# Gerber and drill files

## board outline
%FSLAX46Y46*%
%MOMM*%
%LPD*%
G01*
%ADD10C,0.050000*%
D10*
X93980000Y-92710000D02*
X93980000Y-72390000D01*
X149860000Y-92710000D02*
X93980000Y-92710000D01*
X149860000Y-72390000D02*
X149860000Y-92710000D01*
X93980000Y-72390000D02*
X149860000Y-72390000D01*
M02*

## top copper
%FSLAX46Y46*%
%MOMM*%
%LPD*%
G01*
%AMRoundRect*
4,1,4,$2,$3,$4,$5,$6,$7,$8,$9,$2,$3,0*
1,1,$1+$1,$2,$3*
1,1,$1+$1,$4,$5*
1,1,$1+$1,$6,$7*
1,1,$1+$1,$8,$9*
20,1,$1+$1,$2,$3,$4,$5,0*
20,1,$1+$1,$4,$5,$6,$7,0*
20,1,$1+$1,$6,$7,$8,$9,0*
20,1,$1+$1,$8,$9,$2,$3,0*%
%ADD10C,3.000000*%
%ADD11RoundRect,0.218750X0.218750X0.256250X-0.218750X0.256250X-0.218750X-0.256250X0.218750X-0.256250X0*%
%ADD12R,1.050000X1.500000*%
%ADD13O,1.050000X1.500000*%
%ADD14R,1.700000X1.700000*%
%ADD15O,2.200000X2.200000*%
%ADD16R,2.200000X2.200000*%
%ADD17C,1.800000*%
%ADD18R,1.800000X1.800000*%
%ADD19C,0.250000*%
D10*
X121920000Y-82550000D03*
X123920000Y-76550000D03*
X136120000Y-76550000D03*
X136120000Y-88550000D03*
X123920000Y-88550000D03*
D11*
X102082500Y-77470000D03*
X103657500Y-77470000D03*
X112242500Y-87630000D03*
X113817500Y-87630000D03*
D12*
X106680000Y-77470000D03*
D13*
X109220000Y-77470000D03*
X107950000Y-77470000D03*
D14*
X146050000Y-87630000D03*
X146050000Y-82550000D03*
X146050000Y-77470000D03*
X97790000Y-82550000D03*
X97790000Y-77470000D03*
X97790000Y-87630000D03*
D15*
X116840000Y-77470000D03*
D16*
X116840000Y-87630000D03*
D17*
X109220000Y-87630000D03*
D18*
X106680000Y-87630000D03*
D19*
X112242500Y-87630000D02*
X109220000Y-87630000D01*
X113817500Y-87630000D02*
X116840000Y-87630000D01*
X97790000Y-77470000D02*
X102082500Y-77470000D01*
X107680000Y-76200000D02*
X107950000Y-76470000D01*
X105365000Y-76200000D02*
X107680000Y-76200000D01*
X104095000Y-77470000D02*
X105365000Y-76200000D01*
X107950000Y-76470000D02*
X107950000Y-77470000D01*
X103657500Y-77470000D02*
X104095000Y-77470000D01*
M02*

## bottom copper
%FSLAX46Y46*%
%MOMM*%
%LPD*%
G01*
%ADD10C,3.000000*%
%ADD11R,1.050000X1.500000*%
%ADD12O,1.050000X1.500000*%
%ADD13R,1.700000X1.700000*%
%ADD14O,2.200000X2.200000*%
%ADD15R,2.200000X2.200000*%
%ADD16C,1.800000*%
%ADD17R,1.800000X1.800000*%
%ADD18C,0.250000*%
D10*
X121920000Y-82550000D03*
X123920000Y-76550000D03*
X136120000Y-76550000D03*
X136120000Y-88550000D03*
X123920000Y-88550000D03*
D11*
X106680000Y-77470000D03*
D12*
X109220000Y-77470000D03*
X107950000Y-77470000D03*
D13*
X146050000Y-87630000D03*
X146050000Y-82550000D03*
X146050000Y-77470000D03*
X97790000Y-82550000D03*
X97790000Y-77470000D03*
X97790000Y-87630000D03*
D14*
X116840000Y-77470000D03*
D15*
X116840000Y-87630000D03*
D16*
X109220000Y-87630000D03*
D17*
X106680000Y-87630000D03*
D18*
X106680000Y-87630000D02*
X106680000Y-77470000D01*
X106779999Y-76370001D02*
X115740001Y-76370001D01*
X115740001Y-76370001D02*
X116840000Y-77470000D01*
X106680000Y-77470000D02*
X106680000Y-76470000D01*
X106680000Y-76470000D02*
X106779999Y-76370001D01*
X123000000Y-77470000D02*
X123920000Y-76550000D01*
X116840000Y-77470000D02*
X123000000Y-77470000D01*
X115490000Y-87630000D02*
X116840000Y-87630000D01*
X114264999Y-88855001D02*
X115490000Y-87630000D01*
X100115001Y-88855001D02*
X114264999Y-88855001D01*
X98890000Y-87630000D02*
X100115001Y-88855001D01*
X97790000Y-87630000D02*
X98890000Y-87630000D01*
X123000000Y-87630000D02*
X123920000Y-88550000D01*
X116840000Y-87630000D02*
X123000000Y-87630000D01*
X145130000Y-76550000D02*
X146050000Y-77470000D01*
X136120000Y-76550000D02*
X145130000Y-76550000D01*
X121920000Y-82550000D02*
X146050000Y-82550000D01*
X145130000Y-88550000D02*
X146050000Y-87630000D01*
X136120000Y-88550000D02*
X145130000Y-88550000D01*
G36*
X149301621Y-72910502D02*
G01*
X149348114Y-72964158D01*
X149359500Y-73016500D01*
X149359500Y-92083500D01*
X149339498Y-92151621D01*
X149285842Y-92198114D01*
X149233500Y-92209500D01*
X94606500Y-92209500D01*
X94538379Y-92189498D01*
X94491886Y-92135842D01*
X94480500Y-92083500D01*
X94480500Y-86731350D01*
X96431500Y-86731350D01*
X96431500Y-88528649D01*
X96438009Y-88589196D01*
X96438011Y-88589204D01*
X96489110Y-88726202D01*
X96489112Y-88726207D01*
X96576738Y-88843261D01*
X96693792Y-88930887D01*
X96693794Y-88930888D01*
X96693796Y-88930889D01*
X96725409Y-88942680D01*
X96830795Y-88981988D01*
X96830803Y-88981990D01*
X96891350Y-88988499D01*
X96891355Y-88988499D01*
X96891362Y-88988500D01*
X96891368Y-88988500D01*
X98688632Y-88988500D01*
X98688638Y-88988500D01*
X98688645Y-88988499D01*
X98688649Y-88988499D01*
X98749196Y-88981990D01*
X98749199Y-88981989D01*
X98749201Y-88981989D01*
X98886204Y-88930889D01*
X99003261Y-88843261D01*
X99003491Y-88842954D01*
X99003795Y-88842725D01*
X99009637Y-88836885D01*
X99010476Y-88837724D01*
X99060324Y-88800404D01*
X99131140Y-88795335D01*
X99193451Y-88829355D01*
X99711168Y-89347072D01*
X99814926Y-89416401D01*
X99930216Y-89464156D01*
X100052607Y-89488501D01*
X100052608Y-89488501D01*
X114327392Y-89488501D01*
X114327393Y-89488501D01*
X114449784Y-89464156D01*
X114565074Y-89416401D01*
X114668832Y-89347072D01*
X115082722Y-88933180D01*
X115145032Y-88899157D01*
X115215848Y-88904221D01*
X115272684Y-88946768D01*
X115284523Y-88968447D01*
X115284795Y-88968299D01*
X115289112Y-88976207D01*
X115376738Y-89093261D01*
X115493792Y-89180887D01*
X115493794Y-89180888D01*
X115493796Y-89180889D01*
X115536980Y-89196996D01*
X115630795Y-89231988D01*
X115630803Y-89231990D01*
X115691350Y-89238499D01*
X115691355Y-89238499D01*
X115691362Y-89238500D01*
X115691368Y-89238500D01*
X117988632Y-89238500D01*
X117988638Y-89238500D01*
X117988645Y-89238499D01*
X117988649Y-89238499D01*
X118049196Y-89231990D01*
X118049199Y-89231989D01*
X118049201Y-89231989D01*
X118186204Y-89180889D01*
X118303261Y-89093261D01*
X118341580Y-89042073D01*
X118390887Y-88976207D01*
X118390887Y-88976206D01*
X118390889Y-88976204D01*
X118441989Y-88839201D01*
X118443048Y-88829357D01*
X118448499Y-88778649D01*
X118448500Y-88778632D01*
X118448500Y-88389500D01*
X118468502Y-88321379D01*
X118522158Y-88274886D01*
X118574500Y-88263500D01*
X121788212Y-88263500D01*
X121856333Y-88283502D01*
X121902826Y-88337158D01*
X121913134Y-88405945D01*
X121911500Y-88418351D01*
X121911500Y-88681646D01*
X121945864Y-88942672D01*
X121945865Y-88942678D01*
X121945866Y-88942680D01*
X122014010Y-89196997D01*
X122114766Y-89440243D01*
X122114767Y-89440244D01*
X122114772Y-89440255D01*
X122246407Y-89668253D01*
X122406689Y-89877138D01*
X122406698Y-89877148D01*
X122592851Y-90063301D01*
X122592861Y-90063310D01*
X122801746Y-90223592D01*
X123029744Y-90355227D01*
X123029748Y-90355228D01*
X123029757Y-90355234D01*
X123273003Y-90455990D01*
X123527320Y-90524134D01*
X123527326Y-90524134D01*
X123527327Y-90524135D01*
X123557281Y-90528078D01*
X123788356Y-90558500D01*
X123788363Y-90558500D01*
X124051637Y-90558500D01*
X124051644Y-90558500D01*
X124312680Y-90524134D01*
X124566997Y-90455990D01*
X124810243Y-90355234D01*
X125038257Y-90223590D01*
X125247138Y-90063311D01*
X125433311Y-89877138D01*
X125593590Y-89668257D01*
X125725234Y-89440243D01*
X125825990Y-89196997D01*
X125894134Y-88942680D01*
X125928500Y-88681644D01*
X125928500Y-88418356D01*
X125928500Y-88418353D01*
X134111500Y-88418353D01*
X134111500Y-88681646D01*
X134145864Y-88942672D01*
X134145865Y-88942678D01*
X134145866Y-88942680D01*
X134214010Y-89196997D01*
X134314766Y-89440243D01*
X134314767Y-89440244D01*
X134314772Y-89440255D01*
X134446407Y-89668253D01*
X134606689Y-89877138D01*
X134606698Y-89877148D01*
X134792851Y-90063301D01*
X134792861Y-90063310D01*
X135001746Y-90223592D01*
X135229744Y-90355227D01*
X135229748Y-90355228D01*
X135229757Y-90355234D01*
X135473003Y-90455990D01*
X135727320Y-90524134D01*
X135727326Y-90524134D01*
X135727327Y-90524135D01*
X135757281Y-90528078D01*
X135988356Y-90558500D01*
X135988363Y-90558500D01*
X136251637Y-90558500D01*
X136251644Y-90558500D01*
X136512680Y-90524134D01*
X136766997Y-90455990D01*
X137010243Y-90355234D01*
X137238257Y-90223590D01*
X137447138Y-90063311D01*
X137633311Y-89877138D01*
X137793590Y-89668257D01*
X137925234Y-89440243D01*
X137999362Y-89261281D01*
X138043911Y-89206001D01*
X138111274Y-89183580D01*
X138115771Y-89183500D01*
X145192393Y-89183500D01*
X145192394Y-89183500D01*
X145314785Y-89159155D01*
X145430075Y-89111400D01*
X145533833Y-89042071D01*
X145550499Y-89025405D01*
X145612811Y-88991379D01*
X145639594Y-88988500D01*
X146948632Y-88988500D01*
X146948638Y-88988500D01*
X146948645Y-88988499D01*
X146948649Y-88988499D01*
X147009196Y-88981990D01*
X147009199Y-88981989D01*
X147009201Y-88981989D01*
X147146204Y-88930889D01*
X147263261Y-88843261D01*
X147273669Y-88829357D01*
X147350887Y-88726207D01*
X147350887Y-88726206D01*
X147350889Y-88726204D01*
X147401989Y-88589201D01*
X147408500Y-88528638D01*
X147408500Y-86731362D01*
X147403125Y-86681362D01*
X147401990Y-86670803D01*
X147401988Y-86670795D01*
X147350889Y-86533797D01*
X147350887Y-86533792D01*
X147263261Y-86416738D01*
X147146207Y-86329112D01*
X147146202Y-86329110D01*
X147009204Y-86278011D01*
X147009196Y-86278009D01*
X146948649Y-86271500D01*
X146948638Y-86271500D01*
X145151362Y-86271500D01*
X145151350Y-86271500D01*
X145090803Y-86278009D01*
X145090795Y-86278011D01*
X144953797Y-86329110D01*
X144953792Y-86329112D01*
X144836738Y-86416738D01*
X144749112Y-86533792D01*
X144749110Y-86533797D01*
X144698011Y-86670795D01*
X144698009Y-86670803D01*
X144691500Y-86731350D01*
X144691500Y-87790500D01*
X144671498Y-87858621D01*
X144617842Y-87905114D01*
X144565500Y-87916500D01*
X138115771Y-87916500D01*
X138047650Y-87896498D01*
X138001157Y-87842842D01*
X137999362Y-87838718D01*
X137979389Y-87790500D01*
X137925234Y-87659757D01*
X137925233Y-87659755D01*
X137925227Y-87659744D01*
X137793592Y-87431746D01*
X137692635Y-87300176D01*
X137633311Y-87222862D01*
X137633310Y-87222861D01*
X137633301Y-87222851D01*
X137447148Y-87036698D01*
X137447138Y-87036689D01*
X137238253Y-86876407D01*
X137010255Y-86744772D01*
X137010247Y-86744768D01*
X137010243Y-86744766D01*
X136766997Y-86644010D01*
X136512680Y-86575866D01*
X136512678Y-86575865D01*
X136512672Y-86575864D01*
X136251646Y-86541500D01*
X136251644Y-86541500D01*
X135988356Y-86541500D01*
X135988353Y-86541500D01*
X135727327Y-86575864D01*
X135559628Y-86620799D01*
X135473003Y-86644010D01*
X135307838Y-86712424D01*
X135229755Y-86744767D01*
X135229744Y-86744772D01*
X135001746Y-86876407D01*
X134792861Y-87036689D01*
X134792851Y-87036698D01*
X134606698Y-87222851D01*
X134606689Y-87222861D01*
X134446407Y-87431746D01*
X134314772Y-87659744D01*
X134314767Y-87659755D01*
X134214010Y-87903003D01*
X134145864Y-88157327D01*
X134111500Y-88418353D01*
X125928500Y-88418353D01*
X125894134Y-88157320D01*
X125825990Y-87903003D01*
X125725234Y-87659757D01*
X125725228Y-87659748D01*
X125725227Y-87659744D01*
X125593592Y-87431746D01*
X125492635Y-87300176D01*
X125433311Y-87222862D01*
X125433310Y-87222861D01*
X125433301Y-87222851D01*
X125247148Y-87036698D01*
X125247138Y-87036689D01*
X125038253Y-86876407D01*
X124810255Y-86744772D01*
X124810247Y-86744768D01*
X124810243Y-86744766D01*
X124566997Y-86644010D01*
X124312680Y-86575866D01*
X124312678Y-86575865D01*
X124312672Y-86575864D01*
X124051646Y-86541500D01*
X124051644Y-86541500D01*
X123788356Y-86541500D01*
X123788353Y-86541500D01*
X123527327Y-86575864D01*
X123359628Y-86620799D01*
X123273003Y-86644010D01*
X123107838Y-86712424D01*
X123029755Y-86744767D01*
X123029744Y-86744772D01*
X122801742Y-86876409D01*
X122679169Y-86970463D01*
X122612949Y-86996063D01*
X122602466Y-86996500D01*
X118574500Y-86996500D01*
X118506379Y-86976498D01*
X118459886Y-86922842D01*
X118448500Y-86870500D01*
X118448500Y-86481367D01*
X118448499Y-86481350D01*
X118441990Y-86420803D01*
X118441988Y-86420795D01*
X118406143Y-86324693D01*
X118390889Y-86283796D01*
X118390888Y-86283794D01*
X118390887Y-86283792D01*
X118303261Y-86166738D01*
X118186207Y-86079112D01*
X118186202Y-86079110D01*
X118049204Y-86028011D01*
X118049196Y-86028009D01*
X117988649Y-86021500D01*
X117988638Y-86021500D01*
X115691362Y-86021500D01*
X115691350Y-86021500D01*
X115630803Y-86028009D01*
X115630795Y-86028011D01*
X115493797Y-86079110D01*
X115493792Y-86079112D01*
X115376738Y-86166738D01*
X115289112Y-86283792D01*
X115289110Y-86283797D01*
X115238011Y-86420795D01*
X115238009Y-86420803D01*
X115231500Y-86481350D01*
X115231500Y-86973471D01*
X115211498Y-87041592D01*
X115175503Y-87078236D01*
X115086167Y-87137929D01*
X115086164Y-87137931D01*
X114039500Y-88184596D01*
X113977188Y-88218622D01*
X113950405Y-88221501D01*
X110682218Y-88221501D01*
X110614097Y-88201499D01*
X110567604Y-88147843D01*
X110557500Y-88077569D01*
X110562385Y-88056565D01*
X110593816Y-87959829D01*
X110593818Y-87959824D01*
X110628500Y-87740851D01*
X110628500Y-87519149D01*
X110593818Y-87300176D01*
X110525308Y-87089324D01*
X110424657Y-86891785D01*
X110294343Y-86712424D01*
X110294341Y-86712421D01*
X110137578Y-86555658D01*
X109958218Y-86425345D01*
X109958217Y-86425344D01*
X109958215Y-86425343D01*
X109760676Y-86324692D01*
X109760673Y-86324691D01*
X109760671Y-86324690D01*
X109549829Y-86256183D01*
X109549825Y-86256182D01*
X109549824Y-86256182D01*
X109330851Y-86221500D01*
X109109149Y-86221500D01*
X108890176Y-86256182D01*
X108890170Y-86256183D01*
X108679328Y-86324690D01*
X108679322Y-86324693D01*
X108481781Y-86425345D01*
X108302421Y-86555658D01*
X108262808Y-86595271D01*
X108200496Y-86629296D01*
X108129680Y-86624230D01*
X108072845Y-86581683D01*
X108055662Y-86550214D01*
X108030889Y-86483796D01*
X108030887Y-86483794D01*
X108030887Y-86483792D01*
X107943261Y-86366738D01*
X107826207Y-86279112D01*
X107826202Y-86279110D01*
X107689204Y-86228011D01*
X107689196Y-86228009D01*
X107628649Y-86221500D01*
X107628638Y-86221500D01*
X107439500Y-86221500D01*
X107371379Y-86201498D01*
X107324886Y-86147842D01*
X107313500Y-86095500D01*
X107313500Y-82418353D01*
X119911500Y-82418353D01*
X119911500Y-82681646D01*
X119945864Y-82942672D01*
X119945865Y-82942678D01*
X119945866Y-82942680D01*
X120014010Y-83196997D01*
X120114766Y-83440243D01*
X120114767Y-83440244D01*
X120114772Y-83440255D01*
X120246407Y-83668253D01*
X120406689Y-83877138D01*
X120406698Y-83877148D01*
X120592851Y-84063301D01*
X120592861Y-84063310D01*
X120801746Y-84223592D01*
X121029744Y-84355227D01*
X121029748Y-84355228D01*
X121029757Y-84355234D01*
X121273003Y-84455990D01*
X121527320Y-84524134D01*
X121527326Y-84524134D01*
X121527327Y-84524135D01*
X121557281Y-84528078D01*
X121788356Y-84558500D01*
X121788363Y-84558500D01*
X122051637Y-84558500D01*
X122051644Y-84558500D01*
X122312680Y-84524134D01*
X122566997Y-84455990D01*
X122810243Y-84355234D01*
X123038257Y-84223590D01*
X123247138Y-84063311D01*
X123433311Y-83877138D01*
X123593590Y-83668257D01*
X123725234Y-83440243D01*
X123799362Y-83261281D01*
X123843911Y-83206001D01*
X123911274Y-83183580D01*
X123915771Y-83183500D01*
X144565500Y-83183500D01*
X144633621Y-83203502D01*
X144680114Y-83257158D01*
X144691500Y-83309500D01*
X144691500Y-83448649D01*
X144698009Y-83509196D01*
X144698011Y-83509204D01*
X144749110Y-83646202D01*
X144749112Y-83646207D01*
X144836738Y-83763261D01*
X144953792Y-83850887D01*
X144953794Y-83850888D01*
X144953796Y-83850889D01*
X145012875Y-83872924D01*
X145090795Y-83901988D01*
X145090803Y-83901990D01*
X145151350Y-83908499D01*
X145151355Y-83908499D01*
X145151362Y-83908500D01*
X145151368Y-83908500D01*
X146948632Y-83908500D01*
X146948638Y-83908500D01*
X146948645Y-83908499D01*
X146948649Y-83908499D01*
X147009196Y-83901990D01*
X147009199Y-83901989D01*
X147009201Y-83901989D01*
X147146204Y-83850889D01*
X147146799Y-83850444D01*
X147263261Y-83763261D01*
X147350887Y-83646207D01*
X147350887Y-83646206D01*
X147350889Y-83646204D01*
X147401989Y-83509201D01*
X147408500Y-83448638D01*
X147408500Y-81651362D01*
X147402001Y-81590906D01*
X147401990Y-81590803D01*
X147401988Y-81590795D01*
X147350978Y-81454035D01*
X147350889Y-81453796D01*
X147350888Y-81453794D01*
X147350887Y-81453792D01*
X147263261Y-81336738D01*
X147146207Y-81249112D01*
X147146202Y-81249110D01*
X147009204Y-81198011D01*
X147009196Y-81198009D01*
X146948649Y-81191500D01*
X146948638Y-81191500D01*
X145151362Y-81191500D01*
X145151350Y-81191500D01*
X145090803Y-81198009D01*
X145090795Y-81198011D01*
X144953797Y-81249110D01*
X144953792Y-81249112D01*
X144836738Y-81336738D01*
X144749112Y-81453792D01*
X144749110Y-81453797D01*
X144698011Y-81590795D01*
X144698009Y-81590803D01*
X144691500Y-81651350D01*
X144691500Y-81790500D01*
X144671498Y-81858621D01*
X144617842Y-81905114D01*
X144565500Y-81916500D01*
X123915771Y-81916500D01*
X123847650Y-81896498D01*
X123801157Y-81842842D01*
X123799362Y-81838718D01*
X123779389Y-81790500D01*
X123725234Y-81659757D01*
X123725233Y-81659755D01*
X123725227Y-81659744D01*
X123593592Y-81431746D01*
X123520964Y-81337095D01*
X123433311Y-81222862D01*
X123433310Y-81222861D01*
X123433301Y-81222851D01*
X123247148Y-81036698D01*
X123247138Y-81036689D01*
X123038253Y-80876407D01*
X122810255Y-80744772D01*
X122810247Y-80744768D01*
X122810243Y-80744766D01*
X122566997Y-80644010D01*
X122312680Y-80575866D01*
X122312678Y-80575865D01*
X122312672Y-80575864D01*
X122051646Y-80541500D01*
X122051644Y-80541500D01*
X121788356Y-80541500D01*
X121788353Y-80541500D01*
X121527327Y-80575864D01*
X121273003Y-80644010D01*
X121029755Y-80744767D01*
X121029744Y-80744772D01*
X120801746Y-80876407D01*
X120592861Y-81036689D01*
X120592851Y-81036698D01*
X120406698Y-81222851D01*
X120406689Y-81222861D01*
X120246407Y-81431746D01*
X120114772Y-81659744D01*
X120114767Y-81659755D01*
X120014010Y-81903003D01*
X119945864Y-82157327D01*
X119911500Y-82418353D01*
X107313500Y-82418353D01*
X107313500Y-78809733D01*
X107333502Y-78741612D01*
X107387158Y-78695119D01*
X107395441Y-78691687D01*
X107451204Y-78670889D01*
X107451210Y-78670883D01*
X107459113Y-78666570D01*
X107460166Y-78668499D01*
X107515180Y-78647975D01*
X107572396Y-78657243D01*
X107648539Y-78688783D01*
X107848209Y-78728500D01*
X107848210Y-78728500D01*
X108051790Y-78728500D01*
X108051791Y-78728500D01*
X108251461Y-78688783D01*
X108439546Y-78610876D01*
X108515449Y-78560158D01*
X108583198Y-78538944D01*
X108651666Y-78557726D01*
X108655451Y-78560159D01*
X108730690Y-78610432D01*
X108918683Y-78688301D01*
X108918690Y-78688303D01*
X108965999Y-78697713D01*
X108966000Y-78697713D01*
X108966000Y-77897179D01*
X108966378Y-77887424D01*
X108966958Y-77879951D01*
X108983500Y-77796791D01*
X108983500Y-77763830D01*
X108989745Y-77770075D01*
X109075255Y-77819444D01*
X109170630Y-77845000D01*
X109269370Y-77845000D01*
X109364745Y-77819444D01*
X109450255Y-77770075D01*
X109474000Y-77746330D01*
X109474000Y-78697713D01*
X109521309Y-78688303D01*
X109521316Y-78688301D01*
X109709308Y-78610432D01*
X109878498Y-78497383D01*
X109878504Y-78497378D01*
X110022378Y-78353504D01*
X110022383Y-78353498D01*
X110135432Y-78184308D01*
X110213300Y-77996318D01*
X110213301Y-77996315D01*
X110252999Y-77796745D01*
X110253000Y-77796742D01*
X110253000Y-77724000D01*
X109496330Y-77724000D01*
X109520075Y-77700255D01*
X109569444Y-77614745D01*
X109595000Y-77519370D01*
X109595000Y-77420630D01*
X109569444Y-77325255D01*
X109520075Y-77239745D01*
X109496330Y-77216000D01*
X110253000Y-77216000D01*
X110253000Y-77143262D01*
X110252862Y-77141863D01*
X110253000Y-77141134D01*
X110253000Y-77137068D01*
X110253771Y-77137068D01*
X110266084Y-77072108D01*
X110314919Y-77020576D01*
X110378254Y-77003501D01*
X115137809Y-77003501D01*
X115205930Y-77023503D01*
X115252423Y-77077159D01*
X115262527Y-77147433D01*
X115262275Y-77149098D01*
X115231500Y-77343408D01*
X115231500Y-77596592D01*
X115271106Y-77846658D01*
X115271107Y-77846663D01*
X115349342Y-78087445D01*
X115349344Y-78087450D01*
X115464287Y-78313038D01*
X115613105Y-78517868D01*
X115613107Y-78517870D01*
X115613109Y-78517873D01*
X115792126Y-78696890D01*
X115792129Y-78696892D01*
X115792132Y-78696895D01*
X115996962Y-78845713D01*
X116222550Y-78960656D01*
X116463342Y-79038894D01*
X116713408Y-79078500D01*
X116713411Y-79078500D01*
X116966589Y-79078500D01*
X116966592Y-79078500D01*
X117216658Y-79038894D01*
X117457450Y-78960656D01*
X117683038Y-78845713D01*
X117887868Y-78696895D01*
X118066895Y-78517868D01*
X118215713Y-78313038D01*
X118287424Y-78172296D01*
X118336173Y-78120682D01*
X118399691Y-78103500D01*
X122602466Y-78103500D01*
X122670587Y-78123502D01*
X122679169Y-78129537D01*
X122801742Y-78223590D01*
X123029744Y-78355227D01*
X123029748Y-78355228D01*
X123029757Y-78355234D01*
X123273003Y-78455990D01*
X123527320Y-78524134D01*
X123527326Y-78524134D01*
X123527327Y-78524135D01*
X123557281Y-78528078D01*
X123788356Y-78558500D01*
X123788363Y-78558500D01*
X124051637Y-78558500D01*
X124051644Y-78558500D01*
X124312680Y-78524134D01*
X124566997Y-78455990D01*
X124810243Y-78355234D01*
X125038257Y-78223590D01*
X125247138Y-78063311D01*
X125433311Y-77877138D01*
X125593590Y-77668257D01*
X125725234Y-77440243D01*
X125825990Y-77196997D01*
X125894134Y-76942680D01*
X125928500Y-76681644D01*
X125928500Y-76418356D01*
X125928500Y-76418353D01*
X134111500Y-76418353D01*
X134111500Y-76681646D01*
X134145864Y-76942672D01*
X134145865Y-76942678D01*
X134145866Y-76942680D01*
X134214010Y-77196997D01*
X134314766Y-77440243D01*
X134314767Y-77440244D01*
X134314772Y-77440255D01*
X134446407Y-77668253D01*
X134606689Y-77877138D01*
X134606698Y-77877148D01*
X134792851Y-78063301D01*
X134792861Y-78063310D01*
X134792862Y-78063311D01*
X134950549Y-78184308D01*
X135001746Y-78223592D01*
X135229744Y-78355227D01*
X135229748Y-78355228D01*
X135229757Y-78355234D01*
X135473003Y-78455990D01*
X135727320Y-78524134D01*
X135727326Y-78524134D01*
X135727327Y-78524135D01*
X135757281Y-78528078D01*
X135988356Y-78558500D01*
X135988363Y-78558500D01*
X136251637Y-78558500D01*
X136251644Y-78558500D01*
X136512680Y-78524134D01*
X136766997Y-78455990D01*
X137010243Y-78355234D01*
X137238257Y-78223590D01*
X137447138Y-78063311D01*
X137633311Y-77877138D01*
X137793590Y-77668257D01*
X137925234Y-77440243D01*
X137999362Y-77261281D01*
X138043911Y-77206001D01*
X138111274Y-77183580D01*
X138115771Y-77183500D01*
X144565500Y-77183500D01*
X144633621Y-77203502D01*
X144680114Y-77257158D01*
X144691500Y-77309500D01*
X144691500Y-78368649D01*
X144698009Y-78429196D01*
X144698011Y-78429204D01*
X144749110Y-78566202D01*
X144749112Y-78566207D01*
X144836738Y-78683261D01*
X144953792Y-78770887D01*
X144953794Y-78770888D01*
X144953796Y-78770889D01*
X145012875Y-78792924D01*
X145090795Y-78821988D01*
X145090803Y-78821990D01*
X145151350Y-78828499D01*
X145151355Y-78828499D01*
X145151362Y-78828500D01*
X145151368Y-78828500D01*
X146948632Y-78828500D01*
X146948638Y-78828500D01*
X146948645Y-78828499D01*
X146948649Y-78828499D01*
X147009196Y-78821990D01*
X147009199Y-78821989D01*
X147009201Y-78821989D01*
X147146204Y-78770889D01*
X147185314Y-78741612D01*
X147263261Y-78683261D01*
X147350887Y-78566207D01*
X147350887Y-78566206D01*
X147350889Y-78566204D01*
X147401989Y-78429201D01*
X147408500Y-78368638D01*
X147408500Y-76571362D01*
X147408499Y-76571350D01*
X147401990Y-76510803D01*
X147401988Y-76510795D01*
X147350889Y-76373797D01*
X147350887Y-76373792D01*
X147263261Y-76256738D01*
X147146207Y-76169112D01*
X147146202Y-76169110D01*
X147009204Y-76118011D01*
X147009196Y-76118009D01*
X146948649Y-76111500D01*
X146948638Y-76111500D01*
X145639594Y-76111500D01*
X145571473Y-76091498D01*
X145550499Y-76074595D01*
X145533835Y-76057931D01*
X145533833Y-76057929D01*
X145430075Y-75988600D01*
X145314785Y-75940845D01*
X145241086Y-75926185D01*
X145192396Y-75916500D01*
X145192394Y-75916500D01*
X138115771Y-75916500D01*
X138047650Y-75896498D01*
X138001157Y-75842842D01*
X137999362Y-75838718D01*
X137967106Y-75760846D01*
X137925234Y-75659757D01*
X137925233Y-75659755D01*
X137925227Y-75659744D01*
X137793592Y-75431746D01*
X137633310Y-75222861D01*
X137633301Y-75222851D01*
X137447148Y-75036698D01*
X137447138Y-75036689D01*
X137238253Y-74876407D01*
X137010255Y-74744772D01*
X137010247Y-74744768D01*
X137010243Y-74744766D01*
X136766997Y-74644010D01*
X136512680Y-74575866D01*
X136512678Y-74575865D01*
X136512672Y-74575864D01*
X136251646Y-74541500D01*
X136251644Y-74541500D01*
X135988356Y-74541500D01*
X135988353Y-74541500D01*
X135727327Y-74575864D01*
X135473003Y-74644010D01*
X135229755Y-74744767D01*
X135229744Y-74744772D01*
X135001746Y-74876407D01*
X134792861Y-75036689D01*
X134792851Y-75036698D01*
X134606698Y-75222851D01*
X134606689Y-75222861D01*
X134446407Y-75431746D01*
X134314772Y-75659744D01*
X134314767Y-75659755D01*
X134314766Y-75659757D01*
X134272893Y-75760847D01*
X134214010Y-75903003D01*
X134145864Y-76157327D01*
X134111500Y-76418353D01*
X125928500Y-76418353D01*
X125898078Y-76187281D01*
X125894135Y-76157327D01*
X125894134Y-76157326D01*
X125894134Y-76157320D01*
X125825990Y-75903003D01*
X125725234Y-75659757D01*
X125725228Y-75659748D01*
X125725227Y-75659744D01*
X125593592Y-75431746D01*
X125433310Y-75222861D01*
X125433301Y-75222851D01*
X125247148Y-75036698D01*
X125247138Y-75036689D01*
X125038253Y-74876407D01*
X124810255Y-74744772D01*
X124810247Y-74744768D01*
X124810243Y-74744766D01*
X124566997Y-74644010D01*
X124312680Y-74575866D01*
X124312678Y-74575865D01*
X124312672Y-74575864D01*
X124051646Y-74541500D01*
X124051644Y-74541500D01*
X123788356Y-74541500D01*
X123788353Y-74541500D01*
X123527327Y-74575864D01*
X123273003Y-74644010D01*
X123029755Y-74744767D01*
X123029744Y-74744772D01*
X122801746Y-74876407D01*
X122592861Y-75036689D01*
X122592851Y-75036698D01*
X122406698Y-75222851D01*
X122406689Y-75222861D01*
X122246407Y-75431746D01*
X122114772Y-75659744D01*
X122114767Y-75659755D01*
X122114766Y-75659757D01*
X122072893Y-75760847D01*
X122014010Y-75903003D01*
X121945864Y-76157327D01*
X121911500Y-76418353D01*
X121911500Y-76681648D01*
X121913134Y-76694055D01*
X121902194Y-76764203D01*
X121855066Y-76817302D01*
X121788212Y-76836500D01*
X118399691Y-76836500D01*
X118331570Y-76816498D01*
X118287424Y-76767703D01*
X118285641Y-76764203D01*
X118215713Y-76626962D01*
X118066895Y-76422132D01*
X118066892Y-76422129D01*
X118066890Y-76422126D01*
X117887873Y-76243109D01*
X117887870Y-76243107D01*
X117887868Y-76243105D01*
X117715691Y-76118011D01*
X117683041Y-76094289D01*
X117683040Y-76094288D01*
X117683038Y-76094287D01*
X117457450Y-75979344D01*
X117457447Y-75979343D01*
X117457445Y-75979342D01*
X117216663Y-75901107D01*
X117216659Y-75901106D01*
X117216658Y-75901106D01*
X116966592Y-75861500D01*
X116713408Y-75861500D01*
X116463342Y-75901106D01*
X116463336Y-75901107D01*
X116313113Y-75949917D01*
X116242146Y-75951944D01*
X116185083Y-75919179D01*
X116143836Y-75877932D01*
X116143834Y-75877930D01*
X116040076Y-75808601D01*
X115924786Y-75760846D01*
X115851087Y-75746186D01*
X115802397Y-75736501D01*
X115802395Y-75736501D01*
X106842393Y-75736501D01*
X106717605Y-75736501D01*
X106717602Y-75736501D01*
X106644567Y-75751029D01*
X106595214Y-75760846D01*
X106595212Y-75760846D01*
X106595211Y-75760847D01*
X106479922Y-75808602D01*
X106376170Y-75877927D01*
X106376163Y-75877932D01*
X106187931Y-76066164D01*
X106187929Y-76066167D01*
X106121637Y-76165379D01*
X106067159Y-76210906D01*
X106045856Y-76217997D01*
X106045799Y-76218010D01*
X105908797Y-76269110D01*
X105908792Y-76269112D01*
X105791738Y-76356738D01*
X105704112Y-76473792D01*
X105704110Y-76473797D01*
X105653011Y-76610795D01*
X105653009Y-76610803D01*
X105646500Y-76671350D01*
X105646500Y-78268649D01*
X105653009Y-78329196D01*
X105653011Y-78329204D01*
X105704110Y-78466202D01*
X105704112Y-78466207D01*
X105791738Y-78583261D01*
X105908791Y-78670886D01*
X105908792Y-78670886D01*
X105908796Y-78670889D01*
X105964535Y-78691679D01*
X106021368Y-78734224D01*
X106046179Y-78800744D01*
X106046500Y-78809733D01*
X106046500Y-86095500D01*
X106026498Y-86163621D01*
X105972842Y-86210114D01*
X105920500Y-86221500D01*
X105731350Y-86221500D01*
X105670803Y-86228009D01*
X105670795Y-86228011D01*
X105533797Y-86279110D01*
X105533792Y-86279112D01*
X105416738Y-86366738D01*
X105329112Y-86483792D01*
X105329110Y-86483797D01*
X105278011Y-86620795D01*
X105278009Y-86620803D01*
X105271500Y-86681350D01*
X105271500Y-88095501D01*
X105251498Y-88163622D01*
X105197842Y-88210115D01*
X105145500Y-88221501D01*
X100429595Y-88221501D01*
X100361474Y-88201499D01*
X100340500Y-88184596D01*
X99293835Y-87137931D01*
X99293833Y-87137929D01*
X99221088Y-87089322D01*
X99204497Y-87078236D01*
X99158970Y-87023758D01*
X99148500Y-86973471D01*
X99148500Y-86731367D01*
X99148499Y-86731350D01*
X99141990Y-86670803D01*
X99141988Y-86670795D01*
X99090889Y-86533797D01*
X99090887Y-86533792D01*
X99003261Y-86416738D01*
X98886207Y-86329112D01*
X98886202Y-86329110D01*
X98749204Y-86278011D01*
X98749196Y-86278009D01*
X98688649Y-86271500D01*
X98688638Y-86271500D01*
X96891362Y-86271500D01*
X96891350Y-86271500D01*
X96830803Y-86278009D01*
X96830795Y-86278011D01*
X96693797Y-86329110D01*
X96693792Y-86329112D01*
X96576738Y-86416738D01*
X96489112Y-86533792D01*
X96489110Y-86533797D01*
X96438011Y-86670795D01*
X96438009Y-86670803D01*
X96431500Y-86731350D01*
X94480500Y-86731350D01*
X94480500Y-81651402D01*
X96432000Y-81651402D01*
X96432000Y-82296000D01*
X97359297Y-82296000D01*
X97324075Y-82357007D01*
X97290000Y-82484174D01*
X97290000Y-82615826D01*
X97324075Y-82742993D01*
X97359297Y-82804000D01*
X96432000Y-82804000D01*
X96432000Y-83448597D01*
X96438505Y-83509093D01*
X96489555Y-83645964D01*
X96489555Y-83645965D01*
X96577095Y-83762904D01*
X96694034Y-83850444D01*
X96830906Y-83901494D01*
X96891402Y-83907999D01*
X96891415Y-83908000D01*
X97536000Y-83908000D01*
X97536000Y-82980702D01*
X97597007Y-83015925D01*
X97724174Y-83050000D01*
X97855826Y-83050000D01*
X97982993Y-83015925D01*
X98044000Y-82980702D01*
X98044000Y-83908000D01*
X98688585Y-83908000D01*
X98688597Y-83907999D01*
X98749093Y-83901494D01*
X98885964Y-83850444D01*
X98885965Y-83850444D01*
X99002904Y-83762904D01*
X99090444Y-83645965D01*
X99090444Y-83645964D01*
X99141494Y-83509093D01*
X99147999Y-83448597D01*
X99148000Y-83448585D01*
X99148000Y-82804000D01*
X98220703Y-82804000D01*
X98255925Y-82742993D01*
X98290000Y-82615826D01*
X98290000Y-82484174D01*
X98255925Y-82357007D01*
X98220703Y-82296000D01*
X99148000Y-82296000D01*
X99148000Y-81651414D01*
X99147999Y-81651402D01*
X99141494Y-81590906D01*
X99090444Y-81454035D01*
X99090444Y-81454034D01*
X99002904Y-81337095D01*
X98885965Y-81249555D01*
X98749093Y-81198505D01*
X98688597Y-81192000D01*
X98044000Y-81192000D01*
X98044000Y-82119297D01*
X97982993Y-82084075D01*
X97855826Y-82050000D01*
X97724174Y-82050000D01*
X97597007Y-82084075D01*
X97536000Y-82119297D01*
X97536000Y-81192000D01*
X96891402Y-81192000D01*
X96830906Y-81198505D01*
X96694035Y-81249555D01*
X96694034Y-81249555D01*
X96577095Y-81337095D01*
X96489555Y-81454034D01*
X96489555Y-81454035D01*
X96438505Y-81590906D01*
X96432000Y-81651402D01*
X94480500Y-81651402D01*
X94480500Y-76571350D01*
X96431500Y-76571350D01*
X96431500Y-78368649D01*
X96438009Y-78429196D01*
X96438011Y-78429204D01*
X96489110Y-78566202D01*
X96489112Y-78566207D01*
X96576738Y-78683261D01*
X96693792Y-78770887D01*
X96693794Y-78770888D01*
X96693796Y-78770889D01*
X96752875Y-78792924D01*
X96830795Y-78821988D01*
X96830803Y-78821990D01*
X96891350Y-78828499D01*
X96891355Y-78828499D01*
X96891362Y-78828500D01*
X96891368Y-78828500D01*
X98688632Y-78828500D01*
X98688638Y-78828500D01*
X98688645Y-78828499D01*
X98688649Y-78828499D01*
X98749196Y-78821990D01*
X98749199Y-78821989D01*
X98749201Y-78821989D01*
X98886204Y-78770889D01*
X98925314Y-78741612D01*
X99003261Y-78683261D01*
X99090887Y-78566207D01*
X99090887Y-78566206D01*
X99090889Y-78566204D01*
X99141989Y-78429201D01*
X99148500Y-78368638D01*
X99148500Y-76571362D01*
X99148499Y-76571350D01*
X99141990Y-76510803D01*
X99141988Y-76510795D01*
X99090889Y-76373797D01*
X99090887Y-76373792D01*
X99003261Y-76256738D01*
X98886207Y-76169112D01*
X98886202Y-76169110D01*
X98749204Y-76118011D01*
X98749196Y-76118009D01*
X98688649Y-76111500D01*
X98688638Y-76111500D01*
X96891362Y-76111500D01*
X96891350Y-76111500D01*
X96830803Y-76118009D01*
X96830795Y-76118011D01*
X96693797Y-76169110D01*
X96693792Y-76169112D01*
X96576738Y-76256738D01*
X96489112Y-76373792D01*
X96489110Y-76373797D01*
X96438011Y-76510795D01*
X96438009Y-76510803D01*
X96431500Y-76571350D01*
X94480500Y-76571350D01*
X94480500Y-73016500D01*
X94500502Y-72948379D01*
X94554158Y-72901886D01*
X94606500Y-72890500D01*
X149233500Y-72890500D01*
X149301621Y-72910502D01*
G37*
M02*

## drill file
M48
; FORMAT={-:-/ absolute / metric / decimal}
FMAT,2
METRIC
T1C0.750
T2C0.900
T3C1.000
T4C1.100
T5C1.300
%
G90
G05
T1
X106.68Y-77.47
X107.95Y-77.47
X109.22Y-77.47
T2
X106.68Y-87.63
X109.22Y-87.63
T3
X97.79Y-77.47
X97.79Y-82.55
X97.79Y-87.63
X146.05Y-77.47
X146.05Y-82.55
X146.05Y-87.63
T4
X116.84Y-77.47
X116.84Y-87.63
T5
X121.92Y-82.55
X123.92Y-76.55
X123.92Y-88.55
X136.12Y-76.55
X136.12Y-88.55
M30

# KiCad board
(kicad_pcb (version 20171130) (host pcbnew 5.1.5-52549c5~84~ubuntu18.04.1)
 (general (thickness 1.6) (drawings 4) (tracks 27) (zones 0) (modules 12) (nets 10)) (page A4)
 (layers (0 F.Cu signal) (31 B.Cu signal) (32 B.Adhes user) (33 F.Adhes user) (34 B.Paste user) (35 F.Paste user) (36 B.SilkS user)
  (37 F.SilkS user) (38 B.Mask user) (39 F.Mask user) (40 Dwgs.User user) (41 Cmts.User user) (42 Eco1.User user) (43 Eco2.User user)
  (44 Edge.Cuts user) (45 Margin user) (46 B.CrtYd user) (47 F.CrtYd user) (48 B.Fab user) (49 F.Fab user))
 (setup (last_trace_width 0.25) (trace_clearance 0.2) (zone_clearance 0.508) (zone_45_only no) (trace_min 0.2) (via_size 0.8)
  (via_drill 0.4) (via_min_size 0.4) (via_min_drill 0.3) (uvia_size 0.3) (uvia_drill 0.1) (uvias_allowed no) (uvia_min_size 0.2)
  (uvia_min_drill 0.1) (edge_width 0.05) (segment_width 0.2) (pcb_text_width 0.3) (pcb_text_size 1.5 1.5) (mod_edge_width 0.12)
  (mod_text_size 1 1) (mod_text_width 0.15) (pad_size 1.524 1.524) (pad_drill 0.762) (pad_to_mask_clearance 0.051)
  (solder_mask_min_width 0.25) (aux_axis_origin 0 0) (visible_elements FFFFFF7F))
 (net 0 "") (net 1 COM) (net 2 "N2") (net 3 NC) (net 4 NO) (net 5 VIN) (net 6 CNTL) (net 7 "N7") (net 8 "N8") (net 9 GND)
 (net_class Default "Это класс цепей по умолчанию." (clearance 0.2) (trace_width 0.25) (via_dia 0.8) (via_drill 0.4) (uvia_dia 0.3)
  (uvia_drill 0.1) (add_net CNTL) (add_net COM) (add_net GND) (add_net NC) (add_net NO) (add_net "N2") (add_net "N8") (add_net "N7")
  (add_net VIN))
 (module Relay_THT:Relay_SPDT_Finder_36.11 (layer F.Cu) (at 121.92 82.55)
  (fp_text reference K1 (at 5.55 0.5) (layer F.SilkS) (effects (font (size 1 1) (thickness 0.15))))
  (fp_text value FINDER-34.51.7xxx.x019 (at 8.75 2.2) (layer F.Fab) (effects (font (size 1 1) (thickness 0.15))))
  (pad 11 thru_hole circle (at 0 0) (size 3 3) (drill 1.3) (layers *.Cu *.Mask) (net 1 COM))
  (pad A2 thru_hole circle (at 2 -6) (size 3 3) (drill 1.3) (layers *.Cu *.Mask) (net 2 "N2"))
  (pad 12 thru_hole circle (at 14.2 -6) (size 3 3) (drill 1.3) (layers *.Cu *.Mask) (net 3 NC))
  (pad 14 thru_hole circle (at 14.2 6) (size 3 3) (drill 1.3) (layers *.Cu *.Mask) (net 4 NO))
  (pad A1 thru_hole circle (at 2 6) (size 3 3) (drill 1.3) (layers *.Cu *.Mask) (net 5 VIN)))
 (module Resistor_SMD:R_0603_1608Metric (layer F.Cu) (at 102.87 77.47 180)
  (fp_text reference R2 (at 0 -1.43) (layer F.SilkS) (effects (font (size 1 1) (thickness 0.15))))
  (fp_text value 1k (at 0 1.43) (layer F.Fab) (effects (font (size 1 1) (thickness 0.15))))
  (pad 2 smd roundrect (at 0.7875 0 180) (size 0.875 0.95) (layers F.Cu F.Paste F.Mask) (roundrect_rratio 0.25) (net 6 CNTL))
  (pad 1 smd roundrect (at -0.7875 0 180) (size 0.875 0.95) (layers F.Cu F.Paste F.Mask) (roundrect_rratio 0.25) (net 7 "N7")))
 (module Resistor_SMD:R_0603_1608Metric (layer F.Cu) (at 113.03 87.63 180)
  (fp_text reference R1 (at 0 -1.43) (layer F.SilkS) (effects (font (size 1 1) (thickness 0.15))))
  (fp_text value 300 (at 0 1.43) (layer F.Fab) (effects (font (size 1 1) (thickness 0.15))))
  (pad 2 smd roundrect (at 0.7875 0 180) (size 0.875 0.95) (layers F.Cu F.Paste F.Mask) (roundrect_rratio 0.25) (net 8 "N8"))
  (pad 1 smd roundrect (at -0.7875 0 180) (size 0.875 0.95) (layers F.Cu F.Paste F.Mask) (roundrect_rratio 0.25) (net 5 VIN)))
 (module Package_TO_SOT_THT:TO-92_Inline (layer F.Cu) (at 106.68 77.47)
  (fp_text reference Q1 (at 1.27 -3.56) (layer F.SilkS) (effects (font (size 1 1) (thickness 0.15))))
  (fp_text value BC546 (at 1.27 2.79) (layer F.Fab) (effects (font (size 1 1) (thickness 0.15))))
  (pad 1 thru_hole rect (at 0 0) (size 1.05 1.5) (drill 0.75) (layers *.Cu *.Mask) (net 2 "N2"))
  (pad 3 thru_hole oval (at 2.54 0) (size 1.05 1.5) (drill 0.75) (layers *.Cu *.Mask) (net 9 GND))
  (pad 2 thru_hole oval (at 1.27 0) (size 1.05 1.5) (drill 0.75) (layers *.Cu *.Mask) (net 7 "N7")))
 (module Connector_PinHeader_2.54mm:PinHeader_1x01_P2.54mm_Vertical (layer F.Cu) (at 146.05 87.63)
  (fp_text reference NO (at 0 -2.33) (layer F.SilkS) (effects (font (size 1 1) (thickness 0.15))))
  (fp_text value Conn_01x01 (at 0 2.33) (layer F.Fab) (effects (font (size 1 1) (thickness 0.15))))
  (pad 1 thru_hole rect (at 0 0) (size 1.7 1.7) (drill 1) (layers *.Cu *.Mask) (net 4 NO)))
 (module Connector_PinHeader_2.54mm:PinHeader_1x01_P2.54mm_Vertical (layer F.Cu) (at 146.05 82.55)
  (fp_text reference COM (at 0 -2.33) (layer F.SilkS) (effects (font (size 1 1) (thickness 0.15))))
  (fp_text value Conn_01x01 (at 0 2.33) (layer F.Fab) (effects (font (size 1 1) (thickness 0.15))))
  (pad 1 thru_hole rect (at 0 0) (size 1.7 1.7) (drill 1) (layers *.Cu *.Mask) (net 1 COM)))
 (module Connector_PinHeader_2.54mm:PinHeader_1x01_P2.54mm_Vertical (layer F.Cu) (at 146.05 77.47)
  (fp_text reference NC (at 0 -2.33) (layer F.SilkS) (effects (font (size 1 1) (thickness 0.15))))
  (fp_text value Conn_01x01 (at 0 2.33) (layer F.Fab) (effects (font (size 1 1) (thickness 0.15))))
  (pad 1 thru_hole rect (at 0 0) (size 1.7 1.7) (drill 1) (layers *.Cu *.Mask) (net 3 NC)))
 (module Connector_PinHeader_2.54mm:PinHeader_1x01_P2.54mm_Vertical (layer F.Cu) (at 97.79 82.55)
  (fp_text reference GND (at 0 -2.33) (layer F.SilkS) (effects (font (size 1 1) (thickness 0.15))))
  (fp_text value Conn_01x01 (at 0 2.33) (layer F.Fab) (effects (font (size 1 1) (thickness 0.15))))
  (pad 1 thru_hole rect (at 0 0) (size 1.7 1.7) (drill 1) (layers *.Cu *.Mask) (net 9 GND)))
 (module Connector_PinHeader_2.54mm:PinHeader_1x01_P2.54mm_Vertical (layer F.Cu) (at 97.79 77.47)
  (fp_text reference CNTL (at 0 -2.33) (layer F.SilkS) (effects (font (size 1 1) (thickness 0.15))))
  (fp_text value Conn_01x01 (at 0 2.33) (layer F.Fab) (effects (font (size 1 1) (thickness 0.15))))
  (pad 1 thru_hole rect (at 0 0) (size 1.7 1.7) (drill 1) (layers *.Cu *.Mask) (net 6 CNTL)))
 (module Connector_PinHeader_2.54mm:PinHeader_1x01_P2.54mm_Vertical (layer F.Cu) (at 97.79 87.63)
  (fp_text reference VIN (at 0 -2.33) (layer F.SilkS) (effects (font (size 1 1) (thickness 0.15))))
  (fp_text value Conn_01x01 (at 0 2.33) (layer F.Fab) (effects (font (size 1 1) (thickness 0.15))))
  (pad 1 thru_hole rect (at 0 0) (size 1.7 1.7) (drill 1) (layers *.Cu *.Mask) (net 5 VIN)))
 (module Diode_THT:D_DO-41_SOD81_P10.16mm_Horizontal (layer F.Cu) (at 116.84 87.63 90)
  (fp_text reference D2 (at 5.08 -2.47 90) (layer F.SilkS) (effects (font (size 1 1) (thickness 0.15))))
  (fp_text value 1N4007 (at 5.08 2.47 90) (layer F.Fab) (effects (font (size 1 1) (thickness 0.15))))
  (pad 2 thru_hole oval (at 10.16 0 90) (size 2.2 2.2) (drill 1.1) (layers *.Cu *.Mask) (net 2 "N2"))
  (pad 1 thru_hole rect (at 0 0 90) (size 2.2 2.2) (drill 1.1) (layers *.Cu *.Mask) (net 5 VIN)))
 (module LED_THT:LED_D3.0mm (layer F.Cu) (at 106.68 87.63)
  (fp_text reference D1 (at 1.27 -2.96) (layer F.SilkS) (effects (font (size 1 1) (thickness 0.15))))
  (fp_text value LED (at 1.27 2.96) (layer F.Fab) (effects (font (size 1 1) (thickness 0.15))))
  (pad 2 thru_hole circle (at 2.54 0) (size 1.8 1.8) (drill 0.9) (layers *.Cu *.Mask) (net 8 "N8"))
  (pad 1 thru_hole rect (at 0 0) (size 1.8 1.8) (drill 0.9) (layers *.Cu *.Mask) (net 2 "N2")))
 (gr_line (start 93.98 92.71) (end 93.98 72.39) (layer Edge.Cuts) (width 0.05))
 (gr_line (start 149.86 92.71) (end 93.98 92.71) (layer Edge.Cuts) (width 0.05))
 (gr_line (start 149.86 72.39) (end 149.86 92.71) (layer Edge.Cuts) (width 0.05))
 (gr_line (start 93.98 72.39) (end 149.86 72.39) (layer Edge.Cuts) (width 0.05))
 (segment (start 112.2425 87.63) (end 109.22 87.63) (width 0.25) (layer F.Cu) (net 8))
 (segment (start 106.68 87.63) (end 106.68 77.47) (width 0.25) (layer B.Cu) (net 2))
 (segment (start 106.779999 76.370001) (end 115.740001 76.370001) (width 0.25) (layer B.Cu) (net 2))
 (segment (start 115.740001 76.370001) (end 116.84 77.47) (width 0.25) (layer B.Cu) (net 2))
 (segment (start 106.68 77.47) (end 106.68 76.47) (width 0.25) (layer B.Cu) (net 2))
 (segment (start 106.68 76.47) (end 106.779999 76.370001) (width 0.25) (layer B.Cu) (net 2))
 (segment (start 123 77.47) (end 123.92 76.55) (width 0.25) (layer B.Cu) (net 2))
 (segment (start 116.84 77.47) (end 123 77.47) (width 0.25) (layer B.Cu) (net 2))
 (segment (start 113.8175 87.63) (end 116.84 87.63) (width 0.25) (layer F.Cu) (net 5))
 (segment (start 115.49 87.63) (end 116.84 87.63) (width 0.25) (layer B.Cu) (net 5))
 (segment (start 114.264999 88.855001) (end 115.49 87.63) (width 0.25) (layer B.Cu) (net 5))
 (segment (start 100.115001 88.855001) (end 114.264999 88.855001) (width 0.25) (layer B.Cu) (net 5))
 (segment (start 98.89 87.63) (end 100.115001 88.855001) (width 0.25) (layer B.Cu) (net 5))
 (segment (start 97.79 87.63) (end 98.89 87.63) (width 0.25) (layer B.Cu) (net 5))
 (segment (start 123 87.63) (end 123.92 88.55) (width 0.25) (layer B.Cu) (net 5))
 (segment (start 116.84 87.63) (end 123 87.63) (width 0.25) (layer B.Cu) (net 5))
 (segment (start 97.79 77.47) (end 102.0825 77.47) (width 0.25) (layer F.Cu) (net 6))
 (segment (start 145.13 76.55) (end 146.05 77.47) (width 0.25) (layer B.Cu) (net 3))
 (segment (start 136.12 76.55) (end 145.13 76.55) (width 0.25) (layer B.Cu) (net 3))
 (segment (start 121.92 82.55) (end 146.05 82.55) (width 0.25) (layer B.Cu) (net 1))
 (segment (start 145.13 88.55) (end 146.05 87.63) (width 0.25) (layer B.Cu) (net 4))
 (segment (start 136.12 88.55) (end 145.13 88.55) (width 0.25) (layer B.Cu) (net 4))
 (segment (start 107.68 76.2) (end 107.95 76.47) (width 0.25) (layer F.Cu) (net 7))
 (segment (start 105.365 76.2) (end 107.68 76.2) (width 0.25) (layer F.Cu) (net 7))
 (segment (start 104.095 77.47) (end 105.365 76.2) (width 0.25) (layer F.Cu) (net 7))
 (segment (start 107.95 76.47) (end 107.95 77.47) (width 0.25) (layer F.Cu) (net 7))
 (segment (start 103.6575 77.47) (end 104.095 77.47) (width 0.25) (layer F.Cu) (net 7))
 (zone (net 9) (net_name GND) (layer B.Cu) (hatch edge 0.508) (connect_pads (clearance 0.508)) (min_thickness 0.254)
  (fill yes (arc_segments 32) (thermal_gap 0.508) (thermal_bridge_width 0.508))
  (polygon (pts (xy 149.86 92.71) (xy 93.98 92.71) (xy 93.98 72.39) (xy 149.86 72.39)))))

